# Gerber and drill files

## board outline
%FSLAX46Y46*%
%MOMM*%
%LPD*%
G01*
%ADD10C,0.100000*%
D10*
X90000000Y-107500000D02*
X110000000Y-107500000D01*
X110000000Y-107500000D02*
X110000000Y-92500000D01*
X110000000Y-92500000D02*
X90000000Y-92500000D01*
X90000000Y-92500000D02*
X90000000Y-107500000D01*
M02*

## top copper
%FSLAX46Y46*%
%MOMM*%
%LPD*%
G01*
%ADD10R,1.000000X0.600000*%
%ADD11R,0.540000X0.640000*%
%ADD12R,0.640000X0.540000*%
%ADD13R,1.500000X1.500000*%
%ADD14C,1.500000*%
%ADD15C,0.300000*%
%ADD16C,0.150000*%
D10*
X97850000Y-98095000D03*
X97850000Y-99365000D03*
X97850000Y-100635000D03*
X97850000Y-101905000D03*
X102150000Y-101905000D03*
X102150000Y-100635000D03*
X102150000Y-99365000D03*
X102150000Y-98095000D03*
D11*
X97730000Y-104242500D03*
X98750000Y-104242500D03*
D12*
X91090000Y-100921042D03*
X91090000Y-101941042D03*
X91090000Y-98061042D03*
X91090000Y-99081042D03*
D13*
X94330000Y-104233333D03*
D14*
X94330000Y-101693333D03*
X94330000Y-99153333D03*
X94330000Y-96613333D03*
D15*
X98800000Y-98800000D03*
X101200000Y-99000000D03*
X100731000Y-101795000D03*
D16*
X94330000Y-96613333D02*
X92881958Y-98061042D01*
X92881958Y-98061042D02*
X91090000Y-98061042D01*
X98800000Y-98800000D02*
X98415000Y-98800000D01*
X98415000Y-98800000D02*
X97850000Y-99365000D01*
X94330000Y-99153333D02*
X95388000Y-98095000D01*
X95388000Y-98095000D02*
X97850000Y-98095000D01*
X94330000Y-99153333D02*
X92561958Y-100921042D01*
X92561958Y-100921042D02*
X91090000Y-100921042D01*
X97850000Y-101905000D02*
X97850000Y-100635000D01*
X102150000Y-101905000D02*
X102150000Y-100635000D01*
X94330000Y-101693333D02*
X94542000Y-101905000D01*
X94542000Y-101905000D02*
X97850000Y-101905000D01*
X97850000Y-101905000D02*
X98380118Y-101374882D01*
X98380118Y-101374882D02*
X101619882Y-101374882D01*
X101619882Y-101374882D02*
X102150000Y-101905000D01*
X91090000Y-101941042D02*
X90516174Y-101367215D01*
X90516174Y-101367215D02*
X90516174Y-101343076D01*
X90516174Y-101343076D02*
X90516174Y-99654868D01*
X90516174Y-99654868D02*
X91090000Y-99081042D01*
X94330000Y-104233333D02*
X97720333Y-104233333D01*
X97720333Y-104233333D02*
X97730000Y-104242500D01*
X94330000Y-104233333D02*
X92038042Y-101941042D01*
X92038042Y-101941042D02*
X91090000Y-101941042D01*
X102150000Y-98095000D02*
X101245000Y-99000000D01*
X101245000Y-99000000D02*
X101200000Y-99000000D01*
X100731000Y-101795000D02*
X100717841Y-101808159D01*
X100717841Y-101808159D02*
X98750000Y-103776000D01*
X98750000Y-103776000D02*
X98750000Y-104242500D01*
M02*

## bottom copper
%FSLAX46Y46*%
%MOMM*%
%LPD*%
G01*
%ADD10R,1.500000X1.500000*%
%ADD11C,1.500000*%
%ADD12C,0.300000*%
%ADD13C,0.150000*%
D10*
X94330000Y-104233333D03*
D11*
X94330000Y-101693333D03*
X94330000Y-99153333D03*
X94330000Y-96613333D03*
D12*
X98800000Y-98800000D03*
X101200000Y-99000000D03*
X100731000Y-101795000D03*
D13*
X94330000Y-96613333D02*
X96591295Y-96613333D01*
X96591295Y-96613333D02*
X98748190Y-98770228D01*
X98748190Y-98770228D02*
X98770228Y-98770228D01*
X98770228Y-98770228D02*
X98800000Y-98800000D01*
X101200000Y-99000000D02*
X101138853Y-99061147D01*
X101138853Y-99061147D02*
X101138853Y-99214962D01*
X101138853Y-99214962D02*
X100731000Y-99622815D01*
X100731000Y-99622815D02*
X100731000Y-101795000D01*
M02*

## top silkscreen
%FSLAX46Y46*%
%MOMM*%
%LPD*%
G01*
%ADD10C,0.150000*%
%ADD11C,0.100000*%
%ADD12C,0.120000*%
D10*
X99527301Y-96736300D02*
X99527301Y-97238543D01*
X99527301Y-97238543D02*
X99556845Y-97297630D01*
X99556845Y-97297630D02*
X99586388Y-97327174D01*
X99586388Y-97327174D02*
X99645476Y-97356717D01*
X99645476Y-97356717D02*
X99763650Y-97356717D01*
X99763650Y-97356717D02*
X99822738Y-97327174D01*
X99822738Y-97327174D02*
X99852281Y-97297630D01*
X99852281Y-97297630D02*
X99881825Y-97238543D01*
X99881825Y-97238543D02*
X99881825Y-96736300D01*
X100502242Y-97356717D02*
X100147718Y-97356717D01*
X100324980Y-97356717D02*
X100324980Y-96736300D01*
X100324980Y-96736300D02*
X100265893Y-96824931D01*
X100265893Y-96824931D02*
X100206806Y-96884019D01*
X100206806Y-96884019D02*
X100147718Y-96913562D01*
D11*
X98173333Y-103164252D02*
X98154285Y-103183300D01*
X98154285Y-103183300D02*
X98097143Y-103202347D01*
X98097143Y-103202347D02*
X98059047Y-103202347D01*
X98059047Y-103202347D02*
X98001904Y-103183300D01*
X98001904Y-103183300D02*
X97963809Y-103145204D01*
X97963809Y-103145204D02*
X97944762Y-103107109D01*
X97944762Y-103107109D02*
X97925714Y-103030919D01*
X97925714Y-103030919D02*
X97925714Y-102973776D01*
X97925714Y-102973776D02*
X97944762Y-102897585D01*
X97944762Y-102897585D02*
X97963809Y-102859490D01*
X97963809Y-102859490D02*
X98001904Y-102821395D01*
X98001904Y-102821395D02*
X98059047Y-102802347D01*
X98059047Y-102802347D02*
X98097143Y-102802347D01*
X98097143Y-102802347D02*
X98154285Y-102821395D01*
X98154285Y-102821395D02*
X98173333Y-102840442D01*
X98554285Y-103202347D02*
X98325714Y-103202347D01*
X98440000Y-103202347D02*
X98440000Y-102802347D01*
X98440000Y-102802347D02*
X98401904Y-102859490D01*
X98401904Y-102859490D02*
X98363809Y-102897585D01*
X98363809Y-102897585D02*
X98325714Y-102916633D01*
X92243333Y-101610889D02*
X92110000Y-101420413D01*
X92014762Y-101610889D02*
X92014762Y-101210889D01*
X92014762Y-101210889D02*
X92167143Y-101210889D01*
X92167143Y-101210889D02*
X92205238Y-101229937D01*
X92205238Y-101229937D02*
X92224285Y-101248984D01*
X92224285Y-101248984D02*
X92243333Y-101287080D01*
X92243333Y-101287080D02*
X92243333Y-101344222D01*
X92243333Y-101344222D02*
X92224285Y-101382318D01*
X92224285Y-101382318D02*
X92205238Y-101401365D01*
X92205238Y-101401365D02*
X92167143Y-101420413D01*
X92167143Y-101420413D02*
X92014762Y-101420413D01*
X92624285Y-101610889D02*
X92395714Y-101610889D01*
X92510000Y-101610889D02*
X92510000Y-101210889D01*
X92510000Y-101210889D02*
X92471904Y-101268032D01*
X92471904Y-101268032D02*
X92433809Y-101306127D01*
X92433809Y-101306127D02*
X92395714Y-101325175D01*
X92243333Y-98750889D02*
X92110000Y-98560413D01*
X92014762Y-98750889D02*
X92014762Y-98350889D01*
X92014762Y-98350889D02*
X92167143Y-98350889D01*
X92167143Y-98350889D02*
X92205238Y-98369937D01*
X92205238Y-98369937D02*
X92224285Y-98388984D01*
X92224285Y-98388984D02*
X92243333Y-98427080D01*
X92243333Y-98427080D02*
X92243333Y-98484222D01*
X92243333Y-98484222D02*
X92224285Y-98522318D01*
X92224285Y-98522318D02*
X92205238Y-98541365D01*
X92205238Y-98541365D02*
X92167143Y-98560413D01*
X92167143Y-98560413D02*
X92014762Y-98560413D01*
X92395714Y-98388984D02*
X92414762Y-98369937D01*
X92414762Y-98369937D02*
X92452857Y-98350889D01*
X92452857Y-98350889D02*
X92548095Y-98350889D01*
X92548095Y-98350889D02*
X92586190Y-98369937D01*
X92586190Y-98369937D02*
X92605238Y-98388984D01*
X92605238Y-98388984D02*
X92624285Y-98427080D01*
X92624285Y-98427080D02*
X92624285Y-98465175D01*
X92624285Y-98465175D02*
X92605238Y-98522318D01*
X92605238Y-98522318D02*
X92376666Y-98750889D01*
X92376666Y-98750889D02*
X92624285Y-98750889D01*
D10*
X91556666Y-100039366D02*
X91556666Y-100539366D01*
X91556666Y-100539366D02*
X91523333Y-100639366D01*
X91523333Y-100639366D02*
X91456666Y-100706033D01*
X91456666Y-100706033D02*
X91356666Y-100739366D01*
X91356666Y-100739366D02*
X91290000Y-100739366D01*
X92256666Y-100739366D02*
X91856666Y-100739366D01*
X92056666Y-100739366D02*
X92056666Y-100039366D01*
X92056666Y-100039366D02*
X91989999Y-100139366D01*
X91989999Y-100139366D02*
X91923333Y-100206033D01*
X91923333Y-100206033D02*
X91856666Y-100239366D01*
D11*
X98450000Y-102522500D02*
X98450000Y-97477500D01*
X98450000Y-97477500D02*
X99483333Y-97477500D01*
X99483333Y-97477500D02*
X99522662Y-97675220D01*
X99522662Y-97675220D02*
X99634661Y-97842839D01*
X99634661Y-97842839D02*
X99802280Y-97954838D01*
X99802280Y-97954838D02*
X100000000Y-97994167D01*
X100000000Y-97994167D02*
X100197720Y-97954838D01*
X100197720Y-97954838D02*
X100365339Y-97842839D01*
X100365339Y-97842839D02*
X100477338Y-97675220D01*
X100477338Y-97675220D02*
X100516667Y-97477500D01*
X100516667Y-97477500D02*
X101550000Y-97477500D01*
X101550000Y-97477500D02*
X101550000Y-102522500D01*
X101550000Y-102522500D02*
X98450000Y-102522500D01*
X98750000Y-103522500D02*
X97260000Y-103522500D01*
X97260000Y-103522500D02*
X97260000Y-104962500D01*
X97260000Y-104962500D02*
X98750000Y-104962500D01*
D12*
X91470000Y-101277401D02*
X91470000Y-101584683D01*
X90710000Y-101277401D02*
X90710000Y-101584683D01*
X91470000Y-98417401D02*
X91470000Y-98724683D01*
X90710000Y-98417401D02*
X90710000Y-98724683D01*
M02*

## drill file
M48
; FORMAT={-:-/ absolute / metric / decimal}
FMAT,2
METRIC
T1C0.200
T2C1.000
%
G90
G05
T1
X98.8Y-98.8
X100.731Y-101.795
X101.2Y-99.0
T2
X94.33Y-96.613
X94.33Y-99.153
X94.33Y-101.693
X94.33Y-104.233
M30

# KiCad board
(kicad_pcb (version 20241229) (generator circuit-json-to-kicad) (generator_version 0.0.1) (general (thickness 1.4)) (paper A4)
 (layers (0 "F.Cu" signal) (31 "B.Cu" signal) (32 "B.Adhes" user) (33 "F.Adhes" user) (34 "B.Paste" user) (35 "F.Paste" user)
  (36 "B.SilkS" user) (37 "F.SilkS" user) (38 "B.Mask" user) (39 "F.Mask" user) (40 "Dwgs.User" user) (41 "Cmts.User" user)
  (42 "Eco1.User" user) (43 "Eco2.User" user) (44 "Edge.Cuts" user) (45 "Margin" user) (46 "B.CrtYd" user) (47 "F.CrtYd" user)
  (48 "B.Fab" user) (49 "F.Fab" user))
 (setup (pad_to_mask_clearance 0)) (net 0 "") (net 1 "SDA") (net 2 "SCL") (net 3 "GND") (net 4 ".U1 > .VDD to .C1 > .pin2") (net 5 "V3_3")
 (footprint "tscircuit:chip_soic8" (layer F.Cu) (at 100 100 0)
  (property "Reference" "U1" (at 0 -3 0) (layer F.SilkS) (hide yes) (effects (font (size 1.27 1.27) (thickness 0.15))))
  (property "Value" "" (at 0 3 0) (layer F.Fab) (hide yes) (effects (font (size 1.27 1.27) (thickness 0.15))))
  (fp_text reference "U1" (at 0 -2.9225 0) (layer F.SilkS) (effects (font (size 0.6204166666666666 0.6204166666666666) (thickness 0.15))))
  (fp_line (start -1.5499999999999998 2.5225) (end -1.5499999999999998 -2.5225) (stroke (width 0.1) (type default)) (layer F.SilkS))
  (fp_line (start -1.5499999999999998 -2.5225) (end -0.5166666666666666 -2.5225) (stroke (width 0.1) (type default)) (layer F.SilkS))
  (fp_line (start -0.5166666666666666 -2.5225) (end -0.47733775846416476 -2.32478022661137) (stroke (width 0.1) (type default))
   (layer F.SilkS))
  (fp_line (start -0.47733775846416476 -2.32478022661137) (end -0.3653385036130495 -2.1571614963869505) (stroke (width 0.1) (type default))
   (layer F.SilkS))
  (fp_line (start -0.3653385036130495 -2.1571614963869505) (end -0.19771977338862967 -2.0451622415358353)
   (stroke (width 0.1) (type default)) (layer F.SilkS))
  (fp_line (start -0.19771977338862967 -2.0451622415358353) (end 3.1636708977973285e-17 -2.0058333333333334)
   (stroke (width 0.1) (type default)) (layer F.SilkS))
  (fp_line (start 3.1636708977973285e-17 -2.0058333333333334) (end 0.1977197733886297 -2.0451622415358353)
   (stroke (width 0.1) (type default)) (layer F.SilkS))
  (fp_line (start 0.1977197733886297 -2.0451622415358353) (end 0.3653385036130496 -2.1571614963869505) (stroke (width 0.1) (type default))
   (layer F.SilkS))
  (fp_line (start 0.3653385036130496 -2.1571614963869505) (end 0.47733775846416476 -2.32478022661137) (stroke (width 0.1) (type default))
   (layer F.SilkS))
  (fp_line (start 0.47733775846416476 -2.32478022661137) (end 0.5166666666666666 -2.5225) (stroke (width 0.1) (type default))
   (layer F.SilkS))
  (fp_line (start 0.5166666666666666 -2.5225) (end 1.5499999999999998 -2.5225) (stroke (width 0.1) (type default)) (layer F.SilkS))
  (fp_line (start 1.5499999999999998 -2.5225) (end 1.5499999999999998 2.5225) (stroke (width 0.1) (type default)) (layer F.SilkS))
  (fp_line (start 1.5499999999999998 2.5225) (end -1.5499999999999998 2.5225) (stroke (width 0.1) (type default)) (layer F.SilkS))
  (pad "1" smd rect (at -2.15 -1.905 0) (size 1 0.6) (layers F.Cu F.Paste F.Mask) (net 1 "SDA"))
  (pad "2" smd rect (at -2.15 -0.635 0) (size 1 0.6) (layers F.Cu F.Paste F.Mask) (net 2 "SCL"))
  (pad "3" smd rect (at -2.15 0.635 0) (size 1 0.6) (layers F.Cu F.Paste F.Mask) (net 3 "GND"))
  (pad "4" smd rect (at -2.15 1.905 0) (size 1 0.6) (layers F.Cu F.Paste F.Mask) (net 3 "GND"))
  (pad "5" smd rect (at 2.15 1.905 0) (size 1 0.6) (layers F.Cu F.Paste F.Mask) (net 3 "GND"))
  (pad "6" smd rect (at 2.15 0.635 0) (size 1 0.6) (layers F.Cu F.Paste F.Mask) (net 3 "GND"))
  (pad "7" smd rect (at 2.15 -0.635 0) (size 1 0.6) (layers F.Cu F.Paste F.Mask))
  (pad "8" smd rect (at 2.15 -1.905 0) (size 1 0.6) (layers F.Cu F.Paste F.Mask) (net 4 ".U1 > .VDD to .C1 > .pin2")))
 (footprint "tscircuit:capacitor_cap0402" (layer F.Cu) (at 98.24 104.2425 0)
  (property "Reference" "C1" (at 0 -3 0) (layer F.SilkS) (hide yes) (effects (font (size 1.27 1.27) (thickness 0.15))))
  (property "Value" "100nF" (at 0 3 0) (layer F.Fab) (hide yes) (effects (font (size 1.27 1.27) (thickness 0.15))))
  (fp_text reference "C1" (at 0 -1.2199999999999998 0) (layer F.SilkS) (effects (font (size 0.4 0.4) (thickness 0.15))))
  (fp_line (start 0.51 -0.7199999999999998) (end -0.98 -0.7199999999999998) (stroke (width 0.1) (type default)) (layer F.SilkS))
  (fp_line (start -0.98 -0.7199999999999998) (end -0.98 0.7199999999999998) (stroke (width 0.1) (type default)) (layer F.SilkS))
  (fp_line (start -0.98 0.7199999999999998) (end 0.51 0.7199999999999998) (stroke (width 0.1) (type default)) (layer F.SilkS))
  (pad "1" smd rect (at -0.5100000000000002 0 0) (size 0.54 0.64) (layers F.Cu F.Paste F.Mask) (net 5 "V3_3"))
  (pad "2" smd rect (at 0.51 0 0) (size 0.54 0.64) (layers F.Cu F.Paste F.Mask) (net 4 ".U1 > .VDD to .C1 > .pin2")))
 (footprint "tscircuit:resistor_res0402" (layer F.Cu) (at 91.09 101.43104166666667 -90.00000000000001)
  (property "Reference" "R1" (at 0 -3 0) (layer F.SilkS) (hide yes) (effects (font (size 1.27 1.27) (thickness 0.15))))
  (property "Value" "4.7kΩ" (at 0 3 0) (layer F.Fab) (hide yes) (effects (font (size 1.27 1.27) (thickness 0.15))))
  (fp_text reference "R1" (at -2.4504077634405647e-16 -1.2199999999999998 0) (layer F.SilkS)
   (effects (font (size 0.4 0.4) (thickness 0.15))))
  (fp_line (start -0.15364100000000006 -0.3800000000000007) (end 0.153641 -0.38000000000000084) (stroke (width 0.12) (type default))
   (layer F.SilkS))
  (fp_line (start -0.153641 0.38000000000000084) (end 0.15364100000000006 0.3800000000000007) (stroke (width 0.12) (type default))
   (layer F.SilkS))
  (pad "1" smd rect (at -0.5099999999999999 0 0) (size 0.64 0.54) (layers F.Cu F.Paste F.Mask) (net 1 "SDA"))
  (pad "2" smd rect (at 0.51 0 0) (size 0.64 0.54) (layers F.Cu F.Paste F.Mask) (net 5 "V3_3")))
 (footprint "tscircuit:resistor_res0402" (layer F.Cu) (at 91.09 98.57104166666667 -90.00000000000001)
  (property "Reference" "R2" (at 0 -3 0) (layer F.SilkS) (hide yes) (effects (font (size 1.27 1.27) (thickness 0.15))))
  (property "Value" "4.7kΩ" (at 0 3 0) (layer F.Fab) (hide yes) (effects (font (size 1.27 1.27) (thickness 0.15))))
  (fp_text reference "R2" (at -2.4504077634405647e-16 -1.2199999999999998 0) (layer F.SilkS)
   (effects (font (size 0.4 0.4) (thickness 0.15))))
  (fp_line (start -0.15364100000000006 -0.3800000000000007) (end 0.153641 -0.38000000000000084) (stroke (width 0.12) (type default))
   (layer F.SilkS))
  (fp_line (start -0.153641 0.38000000000000084) (end 0.15364100000000006 0.3800000000000007) (stroke (width 0.12) (type default))
   (layer F.SilkS))
  (pad "1" smd rect (at -0.51 0 0) (size 0.64 0.54) (layers F.Cu F.Paste F.Mask) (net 2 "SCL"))
  (pad "2" smd rect (at 0.5100000000000001 0 0) (size 0.64 0.54) (layers F.Cu F.Paste F.Mask) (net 5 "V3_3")))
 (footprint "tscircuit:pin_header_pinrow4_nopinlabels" (layer F.Cu) (at 94.33 100.42333333333333 90)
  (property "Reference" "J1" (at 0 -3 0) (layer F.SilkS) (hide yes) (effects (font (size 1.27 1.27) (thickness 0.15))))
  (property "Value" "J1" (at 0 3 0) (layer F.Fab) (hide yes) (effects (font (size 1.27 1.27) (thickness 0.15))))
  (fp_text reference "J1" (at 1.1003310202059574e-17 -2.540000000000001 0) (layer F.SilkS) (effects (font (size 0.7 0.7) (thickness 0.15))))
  (pad "1" thru_hole rect (at -3.8100000000000005 2.332952152375708e-16 0) (size 1.5 1.5) (drill 1) (layers *.Cu *.Mask) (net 5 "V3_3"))
  (pad "2" thru_hole circle (at -1.27 7.776507174585693e-17 0) (size 1.5 1.5) (drill 1) (layers *.Cu *.Mask) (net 3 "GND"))
  (pad "3" thru_hole circle (at 1.27 -7.776507174585693e-17 0) (size 1.5 1.5) (drill 1) (layers *.Cu *.Mask) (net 1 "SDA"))
  (pad "4" thru_hole circle (at 3.81 -2.3329521523757077e-16 0) (size 1.5 1.5) (drill 1) (layers *.Cu *.Mask) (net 2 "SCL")))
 (segment (start 94.33 96.61333333333333) (end 92.88195833333333 98.06104166666667) (width 0.15) (layer F.Cu) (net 2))
 (segment (start 92.88195833333333 98.06104166666667) (end 91.09 98.06104166666667) (width 0.15) (layer F.Cu) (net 2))
 (segment (start 94.33 96.61333333333333) (end 96.5912945679117 96.61333333333333) (width 0.15) (layer B.Cu) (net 2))
 (segment (start 96.5912945679117 96.61333333333333) (end 98.74818970635611 98.77022847177776) (width 0.15) (layer B.Cu) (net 2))
 (segment (start 98.74818970635611 98.77022847177776) (end 98.77022847177776 98.77022847177776) (width 0.15) (layer B.Cu) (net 2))
 (segment (start 98.77022847177776 98.77022847177776) (end 98.8 98.8) (width 0.15) (layer B.Cu) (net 2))
 (segment (start 98.8 98.8) (end 98.415 98.8) (width 0.15) (layer F.Cu) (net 2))
 (segment (start 98.415 98.8) (end 97.85 99.365) (width 0.15) (layer F.Cu) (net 2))
 (segment (start 94.33 99.15333333333334) (end 95.388 98.095) (width 0.15) (layer F.Cu) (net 1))
 (segment (start 95.388 98.095) (end 97.85 98.095) (width 0.15) (layer F.Cu) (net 1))
 (segment (start 94.33 99.15333333333334) (end 92.56195833333334 100.92104166666667) (width 0.15) (layer F.Cu) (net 1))
 (segment (start 92.56195833333334 100.92104166666667) (end 91.09 100.92104166666667) (width 0.15) (layer F.Cu) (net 1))
 (segment (start 97.85 101.905) (end 97.85 100.635) (width 0.15) (layer F.Cu) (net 3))
 (segment (start 102.15 101.905) (end 102.15 100.635) (width 0.15) (layer F.Cu) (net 3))
 (segment (start 94.33 101.69333333333333) (end 94.542 101.905) (width 0.15) (layer F.Cu) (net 3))
 (segment (start 94.542 101.905) (end 97.85 101.905) (width 0.15) (layer F.Cu) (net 3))
 (segment (start 97.85 101.905) (end 98.38011811904063 101.37488188095936) (width 0.15) (layer F.Cu) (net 3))
 (segment (start 98.38011811904063 101.37488188095936) (end 101.61988188095937 101.37488188095936) (width 0.15) (layer F.Cu) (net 3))
 (segment (start 101.61988188095937 101.37488188095936) (end 102.15 101.905) (width 0.15) (layer F.Cu) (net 3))
 (segment (start 91.09 101.94104166666666) (end 90.5161737381052 101.36721540477185) (width 0.15) (layer F.Cu) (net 5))
 (segment (start 90.5161737381052 101.36721540477185) (end 90.5161737381052 101.34307551426843) (width 0.15) (layer F.Cu) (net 5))
 (segment (start 90.5161737381052 101.34307551426843) (end 90.5161737381052 99.65486792856147) (width 0.15) (layer F.Cu) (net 5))
 (segment (start 90.5161737381052 99.65486792856147) (end 91.09 99.08104166666666) (width 0.15) (layer F.Cu) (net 5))
 (segment (start 94.33 104.23333333333333) (end 97.72033333333333 104.23333333333333) (width 0.15) (layer F.Cu) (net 5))
 (segment (start 97.72033333333333 104.23333333333333) (end 97.73 104.2425) (width 0.15) (layer F.Cu) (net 5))
 (segment (start 94.33 104.23333333333333) (end 92.03804166666667 101.94104166666666) (width 0.15) (layer F.Cu) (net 5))
 (segment (start 92.03804166666667 101.94104166666666) (end 91.09 101.94104166666666) (width 0.15) (layer F.Cu) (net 5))
 (segment (start 102.15 98.095) (end 101.245 99) (width 0.15) (layer F.Cu) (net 4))
 (segment (start 101.245 99) (end 101.2 99) (width 0.15) (layer F.Cu) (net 4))
 (segment (start 101.2 99) (end 101.1388529808541 99.0611470191459) (width 0.15) (layer B.Cu) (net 4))
 (segment (start 101.1388529808541 99.0611470191459) (end 101.1388529808541 99.21496218480414) (width 0.15) (layer B.Cu) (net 4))
 (segment (start 101.1388529808541 99.21496218480414) (end 100.731 99.62281516565824) (width 0.15) (layer B.Cu) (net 4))
 (segment (start 100.731 99.62281516565824) (end 100.731 101.795) (width 0.15) (layer B.Cu) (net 4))
 (segment (start 100.731 101.795) (end 100.71784144845594 101.80815855154407) (width 0.15) (layer F.Cu) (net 4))
 (segment (start 100.71784144845594 101.80815855154407) (end 98.75 103.776) (width 0.15) (layer F.Cu) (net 4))
 (segment (start 98.75 103.776) (end 98.75 104.2425) (width 0.15) (layer F.Cu) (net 4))
 (gr_line (start 90 107.5) (end 110 107.5) (width 0.1) (layer Edge.Cuts))
 (gr_line (start 110 107.5) (end 110 92.5) (width 0.1) (layer Edge.Cuts))
 (gr_line (start 110 92.5) (end 90 92.5) (width 0.1) (layer Edge.Cuts))
 (gr_line (start 90 92.5) (end 90 107.5) (width 0.1) (layer Edge.Cuts))
 (via (at 98.8 98.8) (size 0.3) (drill 0.2) (layers F.Cu B.Cu) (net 2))
 (via (at 101.2 99) (size 0.3) (drill 0.2) (layers F.Cu B.Cu) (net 4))
 (via (at 100.731 101.795) (size 0.3) (drill 0.2) (layers F.Cu B.Cu) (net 4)))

